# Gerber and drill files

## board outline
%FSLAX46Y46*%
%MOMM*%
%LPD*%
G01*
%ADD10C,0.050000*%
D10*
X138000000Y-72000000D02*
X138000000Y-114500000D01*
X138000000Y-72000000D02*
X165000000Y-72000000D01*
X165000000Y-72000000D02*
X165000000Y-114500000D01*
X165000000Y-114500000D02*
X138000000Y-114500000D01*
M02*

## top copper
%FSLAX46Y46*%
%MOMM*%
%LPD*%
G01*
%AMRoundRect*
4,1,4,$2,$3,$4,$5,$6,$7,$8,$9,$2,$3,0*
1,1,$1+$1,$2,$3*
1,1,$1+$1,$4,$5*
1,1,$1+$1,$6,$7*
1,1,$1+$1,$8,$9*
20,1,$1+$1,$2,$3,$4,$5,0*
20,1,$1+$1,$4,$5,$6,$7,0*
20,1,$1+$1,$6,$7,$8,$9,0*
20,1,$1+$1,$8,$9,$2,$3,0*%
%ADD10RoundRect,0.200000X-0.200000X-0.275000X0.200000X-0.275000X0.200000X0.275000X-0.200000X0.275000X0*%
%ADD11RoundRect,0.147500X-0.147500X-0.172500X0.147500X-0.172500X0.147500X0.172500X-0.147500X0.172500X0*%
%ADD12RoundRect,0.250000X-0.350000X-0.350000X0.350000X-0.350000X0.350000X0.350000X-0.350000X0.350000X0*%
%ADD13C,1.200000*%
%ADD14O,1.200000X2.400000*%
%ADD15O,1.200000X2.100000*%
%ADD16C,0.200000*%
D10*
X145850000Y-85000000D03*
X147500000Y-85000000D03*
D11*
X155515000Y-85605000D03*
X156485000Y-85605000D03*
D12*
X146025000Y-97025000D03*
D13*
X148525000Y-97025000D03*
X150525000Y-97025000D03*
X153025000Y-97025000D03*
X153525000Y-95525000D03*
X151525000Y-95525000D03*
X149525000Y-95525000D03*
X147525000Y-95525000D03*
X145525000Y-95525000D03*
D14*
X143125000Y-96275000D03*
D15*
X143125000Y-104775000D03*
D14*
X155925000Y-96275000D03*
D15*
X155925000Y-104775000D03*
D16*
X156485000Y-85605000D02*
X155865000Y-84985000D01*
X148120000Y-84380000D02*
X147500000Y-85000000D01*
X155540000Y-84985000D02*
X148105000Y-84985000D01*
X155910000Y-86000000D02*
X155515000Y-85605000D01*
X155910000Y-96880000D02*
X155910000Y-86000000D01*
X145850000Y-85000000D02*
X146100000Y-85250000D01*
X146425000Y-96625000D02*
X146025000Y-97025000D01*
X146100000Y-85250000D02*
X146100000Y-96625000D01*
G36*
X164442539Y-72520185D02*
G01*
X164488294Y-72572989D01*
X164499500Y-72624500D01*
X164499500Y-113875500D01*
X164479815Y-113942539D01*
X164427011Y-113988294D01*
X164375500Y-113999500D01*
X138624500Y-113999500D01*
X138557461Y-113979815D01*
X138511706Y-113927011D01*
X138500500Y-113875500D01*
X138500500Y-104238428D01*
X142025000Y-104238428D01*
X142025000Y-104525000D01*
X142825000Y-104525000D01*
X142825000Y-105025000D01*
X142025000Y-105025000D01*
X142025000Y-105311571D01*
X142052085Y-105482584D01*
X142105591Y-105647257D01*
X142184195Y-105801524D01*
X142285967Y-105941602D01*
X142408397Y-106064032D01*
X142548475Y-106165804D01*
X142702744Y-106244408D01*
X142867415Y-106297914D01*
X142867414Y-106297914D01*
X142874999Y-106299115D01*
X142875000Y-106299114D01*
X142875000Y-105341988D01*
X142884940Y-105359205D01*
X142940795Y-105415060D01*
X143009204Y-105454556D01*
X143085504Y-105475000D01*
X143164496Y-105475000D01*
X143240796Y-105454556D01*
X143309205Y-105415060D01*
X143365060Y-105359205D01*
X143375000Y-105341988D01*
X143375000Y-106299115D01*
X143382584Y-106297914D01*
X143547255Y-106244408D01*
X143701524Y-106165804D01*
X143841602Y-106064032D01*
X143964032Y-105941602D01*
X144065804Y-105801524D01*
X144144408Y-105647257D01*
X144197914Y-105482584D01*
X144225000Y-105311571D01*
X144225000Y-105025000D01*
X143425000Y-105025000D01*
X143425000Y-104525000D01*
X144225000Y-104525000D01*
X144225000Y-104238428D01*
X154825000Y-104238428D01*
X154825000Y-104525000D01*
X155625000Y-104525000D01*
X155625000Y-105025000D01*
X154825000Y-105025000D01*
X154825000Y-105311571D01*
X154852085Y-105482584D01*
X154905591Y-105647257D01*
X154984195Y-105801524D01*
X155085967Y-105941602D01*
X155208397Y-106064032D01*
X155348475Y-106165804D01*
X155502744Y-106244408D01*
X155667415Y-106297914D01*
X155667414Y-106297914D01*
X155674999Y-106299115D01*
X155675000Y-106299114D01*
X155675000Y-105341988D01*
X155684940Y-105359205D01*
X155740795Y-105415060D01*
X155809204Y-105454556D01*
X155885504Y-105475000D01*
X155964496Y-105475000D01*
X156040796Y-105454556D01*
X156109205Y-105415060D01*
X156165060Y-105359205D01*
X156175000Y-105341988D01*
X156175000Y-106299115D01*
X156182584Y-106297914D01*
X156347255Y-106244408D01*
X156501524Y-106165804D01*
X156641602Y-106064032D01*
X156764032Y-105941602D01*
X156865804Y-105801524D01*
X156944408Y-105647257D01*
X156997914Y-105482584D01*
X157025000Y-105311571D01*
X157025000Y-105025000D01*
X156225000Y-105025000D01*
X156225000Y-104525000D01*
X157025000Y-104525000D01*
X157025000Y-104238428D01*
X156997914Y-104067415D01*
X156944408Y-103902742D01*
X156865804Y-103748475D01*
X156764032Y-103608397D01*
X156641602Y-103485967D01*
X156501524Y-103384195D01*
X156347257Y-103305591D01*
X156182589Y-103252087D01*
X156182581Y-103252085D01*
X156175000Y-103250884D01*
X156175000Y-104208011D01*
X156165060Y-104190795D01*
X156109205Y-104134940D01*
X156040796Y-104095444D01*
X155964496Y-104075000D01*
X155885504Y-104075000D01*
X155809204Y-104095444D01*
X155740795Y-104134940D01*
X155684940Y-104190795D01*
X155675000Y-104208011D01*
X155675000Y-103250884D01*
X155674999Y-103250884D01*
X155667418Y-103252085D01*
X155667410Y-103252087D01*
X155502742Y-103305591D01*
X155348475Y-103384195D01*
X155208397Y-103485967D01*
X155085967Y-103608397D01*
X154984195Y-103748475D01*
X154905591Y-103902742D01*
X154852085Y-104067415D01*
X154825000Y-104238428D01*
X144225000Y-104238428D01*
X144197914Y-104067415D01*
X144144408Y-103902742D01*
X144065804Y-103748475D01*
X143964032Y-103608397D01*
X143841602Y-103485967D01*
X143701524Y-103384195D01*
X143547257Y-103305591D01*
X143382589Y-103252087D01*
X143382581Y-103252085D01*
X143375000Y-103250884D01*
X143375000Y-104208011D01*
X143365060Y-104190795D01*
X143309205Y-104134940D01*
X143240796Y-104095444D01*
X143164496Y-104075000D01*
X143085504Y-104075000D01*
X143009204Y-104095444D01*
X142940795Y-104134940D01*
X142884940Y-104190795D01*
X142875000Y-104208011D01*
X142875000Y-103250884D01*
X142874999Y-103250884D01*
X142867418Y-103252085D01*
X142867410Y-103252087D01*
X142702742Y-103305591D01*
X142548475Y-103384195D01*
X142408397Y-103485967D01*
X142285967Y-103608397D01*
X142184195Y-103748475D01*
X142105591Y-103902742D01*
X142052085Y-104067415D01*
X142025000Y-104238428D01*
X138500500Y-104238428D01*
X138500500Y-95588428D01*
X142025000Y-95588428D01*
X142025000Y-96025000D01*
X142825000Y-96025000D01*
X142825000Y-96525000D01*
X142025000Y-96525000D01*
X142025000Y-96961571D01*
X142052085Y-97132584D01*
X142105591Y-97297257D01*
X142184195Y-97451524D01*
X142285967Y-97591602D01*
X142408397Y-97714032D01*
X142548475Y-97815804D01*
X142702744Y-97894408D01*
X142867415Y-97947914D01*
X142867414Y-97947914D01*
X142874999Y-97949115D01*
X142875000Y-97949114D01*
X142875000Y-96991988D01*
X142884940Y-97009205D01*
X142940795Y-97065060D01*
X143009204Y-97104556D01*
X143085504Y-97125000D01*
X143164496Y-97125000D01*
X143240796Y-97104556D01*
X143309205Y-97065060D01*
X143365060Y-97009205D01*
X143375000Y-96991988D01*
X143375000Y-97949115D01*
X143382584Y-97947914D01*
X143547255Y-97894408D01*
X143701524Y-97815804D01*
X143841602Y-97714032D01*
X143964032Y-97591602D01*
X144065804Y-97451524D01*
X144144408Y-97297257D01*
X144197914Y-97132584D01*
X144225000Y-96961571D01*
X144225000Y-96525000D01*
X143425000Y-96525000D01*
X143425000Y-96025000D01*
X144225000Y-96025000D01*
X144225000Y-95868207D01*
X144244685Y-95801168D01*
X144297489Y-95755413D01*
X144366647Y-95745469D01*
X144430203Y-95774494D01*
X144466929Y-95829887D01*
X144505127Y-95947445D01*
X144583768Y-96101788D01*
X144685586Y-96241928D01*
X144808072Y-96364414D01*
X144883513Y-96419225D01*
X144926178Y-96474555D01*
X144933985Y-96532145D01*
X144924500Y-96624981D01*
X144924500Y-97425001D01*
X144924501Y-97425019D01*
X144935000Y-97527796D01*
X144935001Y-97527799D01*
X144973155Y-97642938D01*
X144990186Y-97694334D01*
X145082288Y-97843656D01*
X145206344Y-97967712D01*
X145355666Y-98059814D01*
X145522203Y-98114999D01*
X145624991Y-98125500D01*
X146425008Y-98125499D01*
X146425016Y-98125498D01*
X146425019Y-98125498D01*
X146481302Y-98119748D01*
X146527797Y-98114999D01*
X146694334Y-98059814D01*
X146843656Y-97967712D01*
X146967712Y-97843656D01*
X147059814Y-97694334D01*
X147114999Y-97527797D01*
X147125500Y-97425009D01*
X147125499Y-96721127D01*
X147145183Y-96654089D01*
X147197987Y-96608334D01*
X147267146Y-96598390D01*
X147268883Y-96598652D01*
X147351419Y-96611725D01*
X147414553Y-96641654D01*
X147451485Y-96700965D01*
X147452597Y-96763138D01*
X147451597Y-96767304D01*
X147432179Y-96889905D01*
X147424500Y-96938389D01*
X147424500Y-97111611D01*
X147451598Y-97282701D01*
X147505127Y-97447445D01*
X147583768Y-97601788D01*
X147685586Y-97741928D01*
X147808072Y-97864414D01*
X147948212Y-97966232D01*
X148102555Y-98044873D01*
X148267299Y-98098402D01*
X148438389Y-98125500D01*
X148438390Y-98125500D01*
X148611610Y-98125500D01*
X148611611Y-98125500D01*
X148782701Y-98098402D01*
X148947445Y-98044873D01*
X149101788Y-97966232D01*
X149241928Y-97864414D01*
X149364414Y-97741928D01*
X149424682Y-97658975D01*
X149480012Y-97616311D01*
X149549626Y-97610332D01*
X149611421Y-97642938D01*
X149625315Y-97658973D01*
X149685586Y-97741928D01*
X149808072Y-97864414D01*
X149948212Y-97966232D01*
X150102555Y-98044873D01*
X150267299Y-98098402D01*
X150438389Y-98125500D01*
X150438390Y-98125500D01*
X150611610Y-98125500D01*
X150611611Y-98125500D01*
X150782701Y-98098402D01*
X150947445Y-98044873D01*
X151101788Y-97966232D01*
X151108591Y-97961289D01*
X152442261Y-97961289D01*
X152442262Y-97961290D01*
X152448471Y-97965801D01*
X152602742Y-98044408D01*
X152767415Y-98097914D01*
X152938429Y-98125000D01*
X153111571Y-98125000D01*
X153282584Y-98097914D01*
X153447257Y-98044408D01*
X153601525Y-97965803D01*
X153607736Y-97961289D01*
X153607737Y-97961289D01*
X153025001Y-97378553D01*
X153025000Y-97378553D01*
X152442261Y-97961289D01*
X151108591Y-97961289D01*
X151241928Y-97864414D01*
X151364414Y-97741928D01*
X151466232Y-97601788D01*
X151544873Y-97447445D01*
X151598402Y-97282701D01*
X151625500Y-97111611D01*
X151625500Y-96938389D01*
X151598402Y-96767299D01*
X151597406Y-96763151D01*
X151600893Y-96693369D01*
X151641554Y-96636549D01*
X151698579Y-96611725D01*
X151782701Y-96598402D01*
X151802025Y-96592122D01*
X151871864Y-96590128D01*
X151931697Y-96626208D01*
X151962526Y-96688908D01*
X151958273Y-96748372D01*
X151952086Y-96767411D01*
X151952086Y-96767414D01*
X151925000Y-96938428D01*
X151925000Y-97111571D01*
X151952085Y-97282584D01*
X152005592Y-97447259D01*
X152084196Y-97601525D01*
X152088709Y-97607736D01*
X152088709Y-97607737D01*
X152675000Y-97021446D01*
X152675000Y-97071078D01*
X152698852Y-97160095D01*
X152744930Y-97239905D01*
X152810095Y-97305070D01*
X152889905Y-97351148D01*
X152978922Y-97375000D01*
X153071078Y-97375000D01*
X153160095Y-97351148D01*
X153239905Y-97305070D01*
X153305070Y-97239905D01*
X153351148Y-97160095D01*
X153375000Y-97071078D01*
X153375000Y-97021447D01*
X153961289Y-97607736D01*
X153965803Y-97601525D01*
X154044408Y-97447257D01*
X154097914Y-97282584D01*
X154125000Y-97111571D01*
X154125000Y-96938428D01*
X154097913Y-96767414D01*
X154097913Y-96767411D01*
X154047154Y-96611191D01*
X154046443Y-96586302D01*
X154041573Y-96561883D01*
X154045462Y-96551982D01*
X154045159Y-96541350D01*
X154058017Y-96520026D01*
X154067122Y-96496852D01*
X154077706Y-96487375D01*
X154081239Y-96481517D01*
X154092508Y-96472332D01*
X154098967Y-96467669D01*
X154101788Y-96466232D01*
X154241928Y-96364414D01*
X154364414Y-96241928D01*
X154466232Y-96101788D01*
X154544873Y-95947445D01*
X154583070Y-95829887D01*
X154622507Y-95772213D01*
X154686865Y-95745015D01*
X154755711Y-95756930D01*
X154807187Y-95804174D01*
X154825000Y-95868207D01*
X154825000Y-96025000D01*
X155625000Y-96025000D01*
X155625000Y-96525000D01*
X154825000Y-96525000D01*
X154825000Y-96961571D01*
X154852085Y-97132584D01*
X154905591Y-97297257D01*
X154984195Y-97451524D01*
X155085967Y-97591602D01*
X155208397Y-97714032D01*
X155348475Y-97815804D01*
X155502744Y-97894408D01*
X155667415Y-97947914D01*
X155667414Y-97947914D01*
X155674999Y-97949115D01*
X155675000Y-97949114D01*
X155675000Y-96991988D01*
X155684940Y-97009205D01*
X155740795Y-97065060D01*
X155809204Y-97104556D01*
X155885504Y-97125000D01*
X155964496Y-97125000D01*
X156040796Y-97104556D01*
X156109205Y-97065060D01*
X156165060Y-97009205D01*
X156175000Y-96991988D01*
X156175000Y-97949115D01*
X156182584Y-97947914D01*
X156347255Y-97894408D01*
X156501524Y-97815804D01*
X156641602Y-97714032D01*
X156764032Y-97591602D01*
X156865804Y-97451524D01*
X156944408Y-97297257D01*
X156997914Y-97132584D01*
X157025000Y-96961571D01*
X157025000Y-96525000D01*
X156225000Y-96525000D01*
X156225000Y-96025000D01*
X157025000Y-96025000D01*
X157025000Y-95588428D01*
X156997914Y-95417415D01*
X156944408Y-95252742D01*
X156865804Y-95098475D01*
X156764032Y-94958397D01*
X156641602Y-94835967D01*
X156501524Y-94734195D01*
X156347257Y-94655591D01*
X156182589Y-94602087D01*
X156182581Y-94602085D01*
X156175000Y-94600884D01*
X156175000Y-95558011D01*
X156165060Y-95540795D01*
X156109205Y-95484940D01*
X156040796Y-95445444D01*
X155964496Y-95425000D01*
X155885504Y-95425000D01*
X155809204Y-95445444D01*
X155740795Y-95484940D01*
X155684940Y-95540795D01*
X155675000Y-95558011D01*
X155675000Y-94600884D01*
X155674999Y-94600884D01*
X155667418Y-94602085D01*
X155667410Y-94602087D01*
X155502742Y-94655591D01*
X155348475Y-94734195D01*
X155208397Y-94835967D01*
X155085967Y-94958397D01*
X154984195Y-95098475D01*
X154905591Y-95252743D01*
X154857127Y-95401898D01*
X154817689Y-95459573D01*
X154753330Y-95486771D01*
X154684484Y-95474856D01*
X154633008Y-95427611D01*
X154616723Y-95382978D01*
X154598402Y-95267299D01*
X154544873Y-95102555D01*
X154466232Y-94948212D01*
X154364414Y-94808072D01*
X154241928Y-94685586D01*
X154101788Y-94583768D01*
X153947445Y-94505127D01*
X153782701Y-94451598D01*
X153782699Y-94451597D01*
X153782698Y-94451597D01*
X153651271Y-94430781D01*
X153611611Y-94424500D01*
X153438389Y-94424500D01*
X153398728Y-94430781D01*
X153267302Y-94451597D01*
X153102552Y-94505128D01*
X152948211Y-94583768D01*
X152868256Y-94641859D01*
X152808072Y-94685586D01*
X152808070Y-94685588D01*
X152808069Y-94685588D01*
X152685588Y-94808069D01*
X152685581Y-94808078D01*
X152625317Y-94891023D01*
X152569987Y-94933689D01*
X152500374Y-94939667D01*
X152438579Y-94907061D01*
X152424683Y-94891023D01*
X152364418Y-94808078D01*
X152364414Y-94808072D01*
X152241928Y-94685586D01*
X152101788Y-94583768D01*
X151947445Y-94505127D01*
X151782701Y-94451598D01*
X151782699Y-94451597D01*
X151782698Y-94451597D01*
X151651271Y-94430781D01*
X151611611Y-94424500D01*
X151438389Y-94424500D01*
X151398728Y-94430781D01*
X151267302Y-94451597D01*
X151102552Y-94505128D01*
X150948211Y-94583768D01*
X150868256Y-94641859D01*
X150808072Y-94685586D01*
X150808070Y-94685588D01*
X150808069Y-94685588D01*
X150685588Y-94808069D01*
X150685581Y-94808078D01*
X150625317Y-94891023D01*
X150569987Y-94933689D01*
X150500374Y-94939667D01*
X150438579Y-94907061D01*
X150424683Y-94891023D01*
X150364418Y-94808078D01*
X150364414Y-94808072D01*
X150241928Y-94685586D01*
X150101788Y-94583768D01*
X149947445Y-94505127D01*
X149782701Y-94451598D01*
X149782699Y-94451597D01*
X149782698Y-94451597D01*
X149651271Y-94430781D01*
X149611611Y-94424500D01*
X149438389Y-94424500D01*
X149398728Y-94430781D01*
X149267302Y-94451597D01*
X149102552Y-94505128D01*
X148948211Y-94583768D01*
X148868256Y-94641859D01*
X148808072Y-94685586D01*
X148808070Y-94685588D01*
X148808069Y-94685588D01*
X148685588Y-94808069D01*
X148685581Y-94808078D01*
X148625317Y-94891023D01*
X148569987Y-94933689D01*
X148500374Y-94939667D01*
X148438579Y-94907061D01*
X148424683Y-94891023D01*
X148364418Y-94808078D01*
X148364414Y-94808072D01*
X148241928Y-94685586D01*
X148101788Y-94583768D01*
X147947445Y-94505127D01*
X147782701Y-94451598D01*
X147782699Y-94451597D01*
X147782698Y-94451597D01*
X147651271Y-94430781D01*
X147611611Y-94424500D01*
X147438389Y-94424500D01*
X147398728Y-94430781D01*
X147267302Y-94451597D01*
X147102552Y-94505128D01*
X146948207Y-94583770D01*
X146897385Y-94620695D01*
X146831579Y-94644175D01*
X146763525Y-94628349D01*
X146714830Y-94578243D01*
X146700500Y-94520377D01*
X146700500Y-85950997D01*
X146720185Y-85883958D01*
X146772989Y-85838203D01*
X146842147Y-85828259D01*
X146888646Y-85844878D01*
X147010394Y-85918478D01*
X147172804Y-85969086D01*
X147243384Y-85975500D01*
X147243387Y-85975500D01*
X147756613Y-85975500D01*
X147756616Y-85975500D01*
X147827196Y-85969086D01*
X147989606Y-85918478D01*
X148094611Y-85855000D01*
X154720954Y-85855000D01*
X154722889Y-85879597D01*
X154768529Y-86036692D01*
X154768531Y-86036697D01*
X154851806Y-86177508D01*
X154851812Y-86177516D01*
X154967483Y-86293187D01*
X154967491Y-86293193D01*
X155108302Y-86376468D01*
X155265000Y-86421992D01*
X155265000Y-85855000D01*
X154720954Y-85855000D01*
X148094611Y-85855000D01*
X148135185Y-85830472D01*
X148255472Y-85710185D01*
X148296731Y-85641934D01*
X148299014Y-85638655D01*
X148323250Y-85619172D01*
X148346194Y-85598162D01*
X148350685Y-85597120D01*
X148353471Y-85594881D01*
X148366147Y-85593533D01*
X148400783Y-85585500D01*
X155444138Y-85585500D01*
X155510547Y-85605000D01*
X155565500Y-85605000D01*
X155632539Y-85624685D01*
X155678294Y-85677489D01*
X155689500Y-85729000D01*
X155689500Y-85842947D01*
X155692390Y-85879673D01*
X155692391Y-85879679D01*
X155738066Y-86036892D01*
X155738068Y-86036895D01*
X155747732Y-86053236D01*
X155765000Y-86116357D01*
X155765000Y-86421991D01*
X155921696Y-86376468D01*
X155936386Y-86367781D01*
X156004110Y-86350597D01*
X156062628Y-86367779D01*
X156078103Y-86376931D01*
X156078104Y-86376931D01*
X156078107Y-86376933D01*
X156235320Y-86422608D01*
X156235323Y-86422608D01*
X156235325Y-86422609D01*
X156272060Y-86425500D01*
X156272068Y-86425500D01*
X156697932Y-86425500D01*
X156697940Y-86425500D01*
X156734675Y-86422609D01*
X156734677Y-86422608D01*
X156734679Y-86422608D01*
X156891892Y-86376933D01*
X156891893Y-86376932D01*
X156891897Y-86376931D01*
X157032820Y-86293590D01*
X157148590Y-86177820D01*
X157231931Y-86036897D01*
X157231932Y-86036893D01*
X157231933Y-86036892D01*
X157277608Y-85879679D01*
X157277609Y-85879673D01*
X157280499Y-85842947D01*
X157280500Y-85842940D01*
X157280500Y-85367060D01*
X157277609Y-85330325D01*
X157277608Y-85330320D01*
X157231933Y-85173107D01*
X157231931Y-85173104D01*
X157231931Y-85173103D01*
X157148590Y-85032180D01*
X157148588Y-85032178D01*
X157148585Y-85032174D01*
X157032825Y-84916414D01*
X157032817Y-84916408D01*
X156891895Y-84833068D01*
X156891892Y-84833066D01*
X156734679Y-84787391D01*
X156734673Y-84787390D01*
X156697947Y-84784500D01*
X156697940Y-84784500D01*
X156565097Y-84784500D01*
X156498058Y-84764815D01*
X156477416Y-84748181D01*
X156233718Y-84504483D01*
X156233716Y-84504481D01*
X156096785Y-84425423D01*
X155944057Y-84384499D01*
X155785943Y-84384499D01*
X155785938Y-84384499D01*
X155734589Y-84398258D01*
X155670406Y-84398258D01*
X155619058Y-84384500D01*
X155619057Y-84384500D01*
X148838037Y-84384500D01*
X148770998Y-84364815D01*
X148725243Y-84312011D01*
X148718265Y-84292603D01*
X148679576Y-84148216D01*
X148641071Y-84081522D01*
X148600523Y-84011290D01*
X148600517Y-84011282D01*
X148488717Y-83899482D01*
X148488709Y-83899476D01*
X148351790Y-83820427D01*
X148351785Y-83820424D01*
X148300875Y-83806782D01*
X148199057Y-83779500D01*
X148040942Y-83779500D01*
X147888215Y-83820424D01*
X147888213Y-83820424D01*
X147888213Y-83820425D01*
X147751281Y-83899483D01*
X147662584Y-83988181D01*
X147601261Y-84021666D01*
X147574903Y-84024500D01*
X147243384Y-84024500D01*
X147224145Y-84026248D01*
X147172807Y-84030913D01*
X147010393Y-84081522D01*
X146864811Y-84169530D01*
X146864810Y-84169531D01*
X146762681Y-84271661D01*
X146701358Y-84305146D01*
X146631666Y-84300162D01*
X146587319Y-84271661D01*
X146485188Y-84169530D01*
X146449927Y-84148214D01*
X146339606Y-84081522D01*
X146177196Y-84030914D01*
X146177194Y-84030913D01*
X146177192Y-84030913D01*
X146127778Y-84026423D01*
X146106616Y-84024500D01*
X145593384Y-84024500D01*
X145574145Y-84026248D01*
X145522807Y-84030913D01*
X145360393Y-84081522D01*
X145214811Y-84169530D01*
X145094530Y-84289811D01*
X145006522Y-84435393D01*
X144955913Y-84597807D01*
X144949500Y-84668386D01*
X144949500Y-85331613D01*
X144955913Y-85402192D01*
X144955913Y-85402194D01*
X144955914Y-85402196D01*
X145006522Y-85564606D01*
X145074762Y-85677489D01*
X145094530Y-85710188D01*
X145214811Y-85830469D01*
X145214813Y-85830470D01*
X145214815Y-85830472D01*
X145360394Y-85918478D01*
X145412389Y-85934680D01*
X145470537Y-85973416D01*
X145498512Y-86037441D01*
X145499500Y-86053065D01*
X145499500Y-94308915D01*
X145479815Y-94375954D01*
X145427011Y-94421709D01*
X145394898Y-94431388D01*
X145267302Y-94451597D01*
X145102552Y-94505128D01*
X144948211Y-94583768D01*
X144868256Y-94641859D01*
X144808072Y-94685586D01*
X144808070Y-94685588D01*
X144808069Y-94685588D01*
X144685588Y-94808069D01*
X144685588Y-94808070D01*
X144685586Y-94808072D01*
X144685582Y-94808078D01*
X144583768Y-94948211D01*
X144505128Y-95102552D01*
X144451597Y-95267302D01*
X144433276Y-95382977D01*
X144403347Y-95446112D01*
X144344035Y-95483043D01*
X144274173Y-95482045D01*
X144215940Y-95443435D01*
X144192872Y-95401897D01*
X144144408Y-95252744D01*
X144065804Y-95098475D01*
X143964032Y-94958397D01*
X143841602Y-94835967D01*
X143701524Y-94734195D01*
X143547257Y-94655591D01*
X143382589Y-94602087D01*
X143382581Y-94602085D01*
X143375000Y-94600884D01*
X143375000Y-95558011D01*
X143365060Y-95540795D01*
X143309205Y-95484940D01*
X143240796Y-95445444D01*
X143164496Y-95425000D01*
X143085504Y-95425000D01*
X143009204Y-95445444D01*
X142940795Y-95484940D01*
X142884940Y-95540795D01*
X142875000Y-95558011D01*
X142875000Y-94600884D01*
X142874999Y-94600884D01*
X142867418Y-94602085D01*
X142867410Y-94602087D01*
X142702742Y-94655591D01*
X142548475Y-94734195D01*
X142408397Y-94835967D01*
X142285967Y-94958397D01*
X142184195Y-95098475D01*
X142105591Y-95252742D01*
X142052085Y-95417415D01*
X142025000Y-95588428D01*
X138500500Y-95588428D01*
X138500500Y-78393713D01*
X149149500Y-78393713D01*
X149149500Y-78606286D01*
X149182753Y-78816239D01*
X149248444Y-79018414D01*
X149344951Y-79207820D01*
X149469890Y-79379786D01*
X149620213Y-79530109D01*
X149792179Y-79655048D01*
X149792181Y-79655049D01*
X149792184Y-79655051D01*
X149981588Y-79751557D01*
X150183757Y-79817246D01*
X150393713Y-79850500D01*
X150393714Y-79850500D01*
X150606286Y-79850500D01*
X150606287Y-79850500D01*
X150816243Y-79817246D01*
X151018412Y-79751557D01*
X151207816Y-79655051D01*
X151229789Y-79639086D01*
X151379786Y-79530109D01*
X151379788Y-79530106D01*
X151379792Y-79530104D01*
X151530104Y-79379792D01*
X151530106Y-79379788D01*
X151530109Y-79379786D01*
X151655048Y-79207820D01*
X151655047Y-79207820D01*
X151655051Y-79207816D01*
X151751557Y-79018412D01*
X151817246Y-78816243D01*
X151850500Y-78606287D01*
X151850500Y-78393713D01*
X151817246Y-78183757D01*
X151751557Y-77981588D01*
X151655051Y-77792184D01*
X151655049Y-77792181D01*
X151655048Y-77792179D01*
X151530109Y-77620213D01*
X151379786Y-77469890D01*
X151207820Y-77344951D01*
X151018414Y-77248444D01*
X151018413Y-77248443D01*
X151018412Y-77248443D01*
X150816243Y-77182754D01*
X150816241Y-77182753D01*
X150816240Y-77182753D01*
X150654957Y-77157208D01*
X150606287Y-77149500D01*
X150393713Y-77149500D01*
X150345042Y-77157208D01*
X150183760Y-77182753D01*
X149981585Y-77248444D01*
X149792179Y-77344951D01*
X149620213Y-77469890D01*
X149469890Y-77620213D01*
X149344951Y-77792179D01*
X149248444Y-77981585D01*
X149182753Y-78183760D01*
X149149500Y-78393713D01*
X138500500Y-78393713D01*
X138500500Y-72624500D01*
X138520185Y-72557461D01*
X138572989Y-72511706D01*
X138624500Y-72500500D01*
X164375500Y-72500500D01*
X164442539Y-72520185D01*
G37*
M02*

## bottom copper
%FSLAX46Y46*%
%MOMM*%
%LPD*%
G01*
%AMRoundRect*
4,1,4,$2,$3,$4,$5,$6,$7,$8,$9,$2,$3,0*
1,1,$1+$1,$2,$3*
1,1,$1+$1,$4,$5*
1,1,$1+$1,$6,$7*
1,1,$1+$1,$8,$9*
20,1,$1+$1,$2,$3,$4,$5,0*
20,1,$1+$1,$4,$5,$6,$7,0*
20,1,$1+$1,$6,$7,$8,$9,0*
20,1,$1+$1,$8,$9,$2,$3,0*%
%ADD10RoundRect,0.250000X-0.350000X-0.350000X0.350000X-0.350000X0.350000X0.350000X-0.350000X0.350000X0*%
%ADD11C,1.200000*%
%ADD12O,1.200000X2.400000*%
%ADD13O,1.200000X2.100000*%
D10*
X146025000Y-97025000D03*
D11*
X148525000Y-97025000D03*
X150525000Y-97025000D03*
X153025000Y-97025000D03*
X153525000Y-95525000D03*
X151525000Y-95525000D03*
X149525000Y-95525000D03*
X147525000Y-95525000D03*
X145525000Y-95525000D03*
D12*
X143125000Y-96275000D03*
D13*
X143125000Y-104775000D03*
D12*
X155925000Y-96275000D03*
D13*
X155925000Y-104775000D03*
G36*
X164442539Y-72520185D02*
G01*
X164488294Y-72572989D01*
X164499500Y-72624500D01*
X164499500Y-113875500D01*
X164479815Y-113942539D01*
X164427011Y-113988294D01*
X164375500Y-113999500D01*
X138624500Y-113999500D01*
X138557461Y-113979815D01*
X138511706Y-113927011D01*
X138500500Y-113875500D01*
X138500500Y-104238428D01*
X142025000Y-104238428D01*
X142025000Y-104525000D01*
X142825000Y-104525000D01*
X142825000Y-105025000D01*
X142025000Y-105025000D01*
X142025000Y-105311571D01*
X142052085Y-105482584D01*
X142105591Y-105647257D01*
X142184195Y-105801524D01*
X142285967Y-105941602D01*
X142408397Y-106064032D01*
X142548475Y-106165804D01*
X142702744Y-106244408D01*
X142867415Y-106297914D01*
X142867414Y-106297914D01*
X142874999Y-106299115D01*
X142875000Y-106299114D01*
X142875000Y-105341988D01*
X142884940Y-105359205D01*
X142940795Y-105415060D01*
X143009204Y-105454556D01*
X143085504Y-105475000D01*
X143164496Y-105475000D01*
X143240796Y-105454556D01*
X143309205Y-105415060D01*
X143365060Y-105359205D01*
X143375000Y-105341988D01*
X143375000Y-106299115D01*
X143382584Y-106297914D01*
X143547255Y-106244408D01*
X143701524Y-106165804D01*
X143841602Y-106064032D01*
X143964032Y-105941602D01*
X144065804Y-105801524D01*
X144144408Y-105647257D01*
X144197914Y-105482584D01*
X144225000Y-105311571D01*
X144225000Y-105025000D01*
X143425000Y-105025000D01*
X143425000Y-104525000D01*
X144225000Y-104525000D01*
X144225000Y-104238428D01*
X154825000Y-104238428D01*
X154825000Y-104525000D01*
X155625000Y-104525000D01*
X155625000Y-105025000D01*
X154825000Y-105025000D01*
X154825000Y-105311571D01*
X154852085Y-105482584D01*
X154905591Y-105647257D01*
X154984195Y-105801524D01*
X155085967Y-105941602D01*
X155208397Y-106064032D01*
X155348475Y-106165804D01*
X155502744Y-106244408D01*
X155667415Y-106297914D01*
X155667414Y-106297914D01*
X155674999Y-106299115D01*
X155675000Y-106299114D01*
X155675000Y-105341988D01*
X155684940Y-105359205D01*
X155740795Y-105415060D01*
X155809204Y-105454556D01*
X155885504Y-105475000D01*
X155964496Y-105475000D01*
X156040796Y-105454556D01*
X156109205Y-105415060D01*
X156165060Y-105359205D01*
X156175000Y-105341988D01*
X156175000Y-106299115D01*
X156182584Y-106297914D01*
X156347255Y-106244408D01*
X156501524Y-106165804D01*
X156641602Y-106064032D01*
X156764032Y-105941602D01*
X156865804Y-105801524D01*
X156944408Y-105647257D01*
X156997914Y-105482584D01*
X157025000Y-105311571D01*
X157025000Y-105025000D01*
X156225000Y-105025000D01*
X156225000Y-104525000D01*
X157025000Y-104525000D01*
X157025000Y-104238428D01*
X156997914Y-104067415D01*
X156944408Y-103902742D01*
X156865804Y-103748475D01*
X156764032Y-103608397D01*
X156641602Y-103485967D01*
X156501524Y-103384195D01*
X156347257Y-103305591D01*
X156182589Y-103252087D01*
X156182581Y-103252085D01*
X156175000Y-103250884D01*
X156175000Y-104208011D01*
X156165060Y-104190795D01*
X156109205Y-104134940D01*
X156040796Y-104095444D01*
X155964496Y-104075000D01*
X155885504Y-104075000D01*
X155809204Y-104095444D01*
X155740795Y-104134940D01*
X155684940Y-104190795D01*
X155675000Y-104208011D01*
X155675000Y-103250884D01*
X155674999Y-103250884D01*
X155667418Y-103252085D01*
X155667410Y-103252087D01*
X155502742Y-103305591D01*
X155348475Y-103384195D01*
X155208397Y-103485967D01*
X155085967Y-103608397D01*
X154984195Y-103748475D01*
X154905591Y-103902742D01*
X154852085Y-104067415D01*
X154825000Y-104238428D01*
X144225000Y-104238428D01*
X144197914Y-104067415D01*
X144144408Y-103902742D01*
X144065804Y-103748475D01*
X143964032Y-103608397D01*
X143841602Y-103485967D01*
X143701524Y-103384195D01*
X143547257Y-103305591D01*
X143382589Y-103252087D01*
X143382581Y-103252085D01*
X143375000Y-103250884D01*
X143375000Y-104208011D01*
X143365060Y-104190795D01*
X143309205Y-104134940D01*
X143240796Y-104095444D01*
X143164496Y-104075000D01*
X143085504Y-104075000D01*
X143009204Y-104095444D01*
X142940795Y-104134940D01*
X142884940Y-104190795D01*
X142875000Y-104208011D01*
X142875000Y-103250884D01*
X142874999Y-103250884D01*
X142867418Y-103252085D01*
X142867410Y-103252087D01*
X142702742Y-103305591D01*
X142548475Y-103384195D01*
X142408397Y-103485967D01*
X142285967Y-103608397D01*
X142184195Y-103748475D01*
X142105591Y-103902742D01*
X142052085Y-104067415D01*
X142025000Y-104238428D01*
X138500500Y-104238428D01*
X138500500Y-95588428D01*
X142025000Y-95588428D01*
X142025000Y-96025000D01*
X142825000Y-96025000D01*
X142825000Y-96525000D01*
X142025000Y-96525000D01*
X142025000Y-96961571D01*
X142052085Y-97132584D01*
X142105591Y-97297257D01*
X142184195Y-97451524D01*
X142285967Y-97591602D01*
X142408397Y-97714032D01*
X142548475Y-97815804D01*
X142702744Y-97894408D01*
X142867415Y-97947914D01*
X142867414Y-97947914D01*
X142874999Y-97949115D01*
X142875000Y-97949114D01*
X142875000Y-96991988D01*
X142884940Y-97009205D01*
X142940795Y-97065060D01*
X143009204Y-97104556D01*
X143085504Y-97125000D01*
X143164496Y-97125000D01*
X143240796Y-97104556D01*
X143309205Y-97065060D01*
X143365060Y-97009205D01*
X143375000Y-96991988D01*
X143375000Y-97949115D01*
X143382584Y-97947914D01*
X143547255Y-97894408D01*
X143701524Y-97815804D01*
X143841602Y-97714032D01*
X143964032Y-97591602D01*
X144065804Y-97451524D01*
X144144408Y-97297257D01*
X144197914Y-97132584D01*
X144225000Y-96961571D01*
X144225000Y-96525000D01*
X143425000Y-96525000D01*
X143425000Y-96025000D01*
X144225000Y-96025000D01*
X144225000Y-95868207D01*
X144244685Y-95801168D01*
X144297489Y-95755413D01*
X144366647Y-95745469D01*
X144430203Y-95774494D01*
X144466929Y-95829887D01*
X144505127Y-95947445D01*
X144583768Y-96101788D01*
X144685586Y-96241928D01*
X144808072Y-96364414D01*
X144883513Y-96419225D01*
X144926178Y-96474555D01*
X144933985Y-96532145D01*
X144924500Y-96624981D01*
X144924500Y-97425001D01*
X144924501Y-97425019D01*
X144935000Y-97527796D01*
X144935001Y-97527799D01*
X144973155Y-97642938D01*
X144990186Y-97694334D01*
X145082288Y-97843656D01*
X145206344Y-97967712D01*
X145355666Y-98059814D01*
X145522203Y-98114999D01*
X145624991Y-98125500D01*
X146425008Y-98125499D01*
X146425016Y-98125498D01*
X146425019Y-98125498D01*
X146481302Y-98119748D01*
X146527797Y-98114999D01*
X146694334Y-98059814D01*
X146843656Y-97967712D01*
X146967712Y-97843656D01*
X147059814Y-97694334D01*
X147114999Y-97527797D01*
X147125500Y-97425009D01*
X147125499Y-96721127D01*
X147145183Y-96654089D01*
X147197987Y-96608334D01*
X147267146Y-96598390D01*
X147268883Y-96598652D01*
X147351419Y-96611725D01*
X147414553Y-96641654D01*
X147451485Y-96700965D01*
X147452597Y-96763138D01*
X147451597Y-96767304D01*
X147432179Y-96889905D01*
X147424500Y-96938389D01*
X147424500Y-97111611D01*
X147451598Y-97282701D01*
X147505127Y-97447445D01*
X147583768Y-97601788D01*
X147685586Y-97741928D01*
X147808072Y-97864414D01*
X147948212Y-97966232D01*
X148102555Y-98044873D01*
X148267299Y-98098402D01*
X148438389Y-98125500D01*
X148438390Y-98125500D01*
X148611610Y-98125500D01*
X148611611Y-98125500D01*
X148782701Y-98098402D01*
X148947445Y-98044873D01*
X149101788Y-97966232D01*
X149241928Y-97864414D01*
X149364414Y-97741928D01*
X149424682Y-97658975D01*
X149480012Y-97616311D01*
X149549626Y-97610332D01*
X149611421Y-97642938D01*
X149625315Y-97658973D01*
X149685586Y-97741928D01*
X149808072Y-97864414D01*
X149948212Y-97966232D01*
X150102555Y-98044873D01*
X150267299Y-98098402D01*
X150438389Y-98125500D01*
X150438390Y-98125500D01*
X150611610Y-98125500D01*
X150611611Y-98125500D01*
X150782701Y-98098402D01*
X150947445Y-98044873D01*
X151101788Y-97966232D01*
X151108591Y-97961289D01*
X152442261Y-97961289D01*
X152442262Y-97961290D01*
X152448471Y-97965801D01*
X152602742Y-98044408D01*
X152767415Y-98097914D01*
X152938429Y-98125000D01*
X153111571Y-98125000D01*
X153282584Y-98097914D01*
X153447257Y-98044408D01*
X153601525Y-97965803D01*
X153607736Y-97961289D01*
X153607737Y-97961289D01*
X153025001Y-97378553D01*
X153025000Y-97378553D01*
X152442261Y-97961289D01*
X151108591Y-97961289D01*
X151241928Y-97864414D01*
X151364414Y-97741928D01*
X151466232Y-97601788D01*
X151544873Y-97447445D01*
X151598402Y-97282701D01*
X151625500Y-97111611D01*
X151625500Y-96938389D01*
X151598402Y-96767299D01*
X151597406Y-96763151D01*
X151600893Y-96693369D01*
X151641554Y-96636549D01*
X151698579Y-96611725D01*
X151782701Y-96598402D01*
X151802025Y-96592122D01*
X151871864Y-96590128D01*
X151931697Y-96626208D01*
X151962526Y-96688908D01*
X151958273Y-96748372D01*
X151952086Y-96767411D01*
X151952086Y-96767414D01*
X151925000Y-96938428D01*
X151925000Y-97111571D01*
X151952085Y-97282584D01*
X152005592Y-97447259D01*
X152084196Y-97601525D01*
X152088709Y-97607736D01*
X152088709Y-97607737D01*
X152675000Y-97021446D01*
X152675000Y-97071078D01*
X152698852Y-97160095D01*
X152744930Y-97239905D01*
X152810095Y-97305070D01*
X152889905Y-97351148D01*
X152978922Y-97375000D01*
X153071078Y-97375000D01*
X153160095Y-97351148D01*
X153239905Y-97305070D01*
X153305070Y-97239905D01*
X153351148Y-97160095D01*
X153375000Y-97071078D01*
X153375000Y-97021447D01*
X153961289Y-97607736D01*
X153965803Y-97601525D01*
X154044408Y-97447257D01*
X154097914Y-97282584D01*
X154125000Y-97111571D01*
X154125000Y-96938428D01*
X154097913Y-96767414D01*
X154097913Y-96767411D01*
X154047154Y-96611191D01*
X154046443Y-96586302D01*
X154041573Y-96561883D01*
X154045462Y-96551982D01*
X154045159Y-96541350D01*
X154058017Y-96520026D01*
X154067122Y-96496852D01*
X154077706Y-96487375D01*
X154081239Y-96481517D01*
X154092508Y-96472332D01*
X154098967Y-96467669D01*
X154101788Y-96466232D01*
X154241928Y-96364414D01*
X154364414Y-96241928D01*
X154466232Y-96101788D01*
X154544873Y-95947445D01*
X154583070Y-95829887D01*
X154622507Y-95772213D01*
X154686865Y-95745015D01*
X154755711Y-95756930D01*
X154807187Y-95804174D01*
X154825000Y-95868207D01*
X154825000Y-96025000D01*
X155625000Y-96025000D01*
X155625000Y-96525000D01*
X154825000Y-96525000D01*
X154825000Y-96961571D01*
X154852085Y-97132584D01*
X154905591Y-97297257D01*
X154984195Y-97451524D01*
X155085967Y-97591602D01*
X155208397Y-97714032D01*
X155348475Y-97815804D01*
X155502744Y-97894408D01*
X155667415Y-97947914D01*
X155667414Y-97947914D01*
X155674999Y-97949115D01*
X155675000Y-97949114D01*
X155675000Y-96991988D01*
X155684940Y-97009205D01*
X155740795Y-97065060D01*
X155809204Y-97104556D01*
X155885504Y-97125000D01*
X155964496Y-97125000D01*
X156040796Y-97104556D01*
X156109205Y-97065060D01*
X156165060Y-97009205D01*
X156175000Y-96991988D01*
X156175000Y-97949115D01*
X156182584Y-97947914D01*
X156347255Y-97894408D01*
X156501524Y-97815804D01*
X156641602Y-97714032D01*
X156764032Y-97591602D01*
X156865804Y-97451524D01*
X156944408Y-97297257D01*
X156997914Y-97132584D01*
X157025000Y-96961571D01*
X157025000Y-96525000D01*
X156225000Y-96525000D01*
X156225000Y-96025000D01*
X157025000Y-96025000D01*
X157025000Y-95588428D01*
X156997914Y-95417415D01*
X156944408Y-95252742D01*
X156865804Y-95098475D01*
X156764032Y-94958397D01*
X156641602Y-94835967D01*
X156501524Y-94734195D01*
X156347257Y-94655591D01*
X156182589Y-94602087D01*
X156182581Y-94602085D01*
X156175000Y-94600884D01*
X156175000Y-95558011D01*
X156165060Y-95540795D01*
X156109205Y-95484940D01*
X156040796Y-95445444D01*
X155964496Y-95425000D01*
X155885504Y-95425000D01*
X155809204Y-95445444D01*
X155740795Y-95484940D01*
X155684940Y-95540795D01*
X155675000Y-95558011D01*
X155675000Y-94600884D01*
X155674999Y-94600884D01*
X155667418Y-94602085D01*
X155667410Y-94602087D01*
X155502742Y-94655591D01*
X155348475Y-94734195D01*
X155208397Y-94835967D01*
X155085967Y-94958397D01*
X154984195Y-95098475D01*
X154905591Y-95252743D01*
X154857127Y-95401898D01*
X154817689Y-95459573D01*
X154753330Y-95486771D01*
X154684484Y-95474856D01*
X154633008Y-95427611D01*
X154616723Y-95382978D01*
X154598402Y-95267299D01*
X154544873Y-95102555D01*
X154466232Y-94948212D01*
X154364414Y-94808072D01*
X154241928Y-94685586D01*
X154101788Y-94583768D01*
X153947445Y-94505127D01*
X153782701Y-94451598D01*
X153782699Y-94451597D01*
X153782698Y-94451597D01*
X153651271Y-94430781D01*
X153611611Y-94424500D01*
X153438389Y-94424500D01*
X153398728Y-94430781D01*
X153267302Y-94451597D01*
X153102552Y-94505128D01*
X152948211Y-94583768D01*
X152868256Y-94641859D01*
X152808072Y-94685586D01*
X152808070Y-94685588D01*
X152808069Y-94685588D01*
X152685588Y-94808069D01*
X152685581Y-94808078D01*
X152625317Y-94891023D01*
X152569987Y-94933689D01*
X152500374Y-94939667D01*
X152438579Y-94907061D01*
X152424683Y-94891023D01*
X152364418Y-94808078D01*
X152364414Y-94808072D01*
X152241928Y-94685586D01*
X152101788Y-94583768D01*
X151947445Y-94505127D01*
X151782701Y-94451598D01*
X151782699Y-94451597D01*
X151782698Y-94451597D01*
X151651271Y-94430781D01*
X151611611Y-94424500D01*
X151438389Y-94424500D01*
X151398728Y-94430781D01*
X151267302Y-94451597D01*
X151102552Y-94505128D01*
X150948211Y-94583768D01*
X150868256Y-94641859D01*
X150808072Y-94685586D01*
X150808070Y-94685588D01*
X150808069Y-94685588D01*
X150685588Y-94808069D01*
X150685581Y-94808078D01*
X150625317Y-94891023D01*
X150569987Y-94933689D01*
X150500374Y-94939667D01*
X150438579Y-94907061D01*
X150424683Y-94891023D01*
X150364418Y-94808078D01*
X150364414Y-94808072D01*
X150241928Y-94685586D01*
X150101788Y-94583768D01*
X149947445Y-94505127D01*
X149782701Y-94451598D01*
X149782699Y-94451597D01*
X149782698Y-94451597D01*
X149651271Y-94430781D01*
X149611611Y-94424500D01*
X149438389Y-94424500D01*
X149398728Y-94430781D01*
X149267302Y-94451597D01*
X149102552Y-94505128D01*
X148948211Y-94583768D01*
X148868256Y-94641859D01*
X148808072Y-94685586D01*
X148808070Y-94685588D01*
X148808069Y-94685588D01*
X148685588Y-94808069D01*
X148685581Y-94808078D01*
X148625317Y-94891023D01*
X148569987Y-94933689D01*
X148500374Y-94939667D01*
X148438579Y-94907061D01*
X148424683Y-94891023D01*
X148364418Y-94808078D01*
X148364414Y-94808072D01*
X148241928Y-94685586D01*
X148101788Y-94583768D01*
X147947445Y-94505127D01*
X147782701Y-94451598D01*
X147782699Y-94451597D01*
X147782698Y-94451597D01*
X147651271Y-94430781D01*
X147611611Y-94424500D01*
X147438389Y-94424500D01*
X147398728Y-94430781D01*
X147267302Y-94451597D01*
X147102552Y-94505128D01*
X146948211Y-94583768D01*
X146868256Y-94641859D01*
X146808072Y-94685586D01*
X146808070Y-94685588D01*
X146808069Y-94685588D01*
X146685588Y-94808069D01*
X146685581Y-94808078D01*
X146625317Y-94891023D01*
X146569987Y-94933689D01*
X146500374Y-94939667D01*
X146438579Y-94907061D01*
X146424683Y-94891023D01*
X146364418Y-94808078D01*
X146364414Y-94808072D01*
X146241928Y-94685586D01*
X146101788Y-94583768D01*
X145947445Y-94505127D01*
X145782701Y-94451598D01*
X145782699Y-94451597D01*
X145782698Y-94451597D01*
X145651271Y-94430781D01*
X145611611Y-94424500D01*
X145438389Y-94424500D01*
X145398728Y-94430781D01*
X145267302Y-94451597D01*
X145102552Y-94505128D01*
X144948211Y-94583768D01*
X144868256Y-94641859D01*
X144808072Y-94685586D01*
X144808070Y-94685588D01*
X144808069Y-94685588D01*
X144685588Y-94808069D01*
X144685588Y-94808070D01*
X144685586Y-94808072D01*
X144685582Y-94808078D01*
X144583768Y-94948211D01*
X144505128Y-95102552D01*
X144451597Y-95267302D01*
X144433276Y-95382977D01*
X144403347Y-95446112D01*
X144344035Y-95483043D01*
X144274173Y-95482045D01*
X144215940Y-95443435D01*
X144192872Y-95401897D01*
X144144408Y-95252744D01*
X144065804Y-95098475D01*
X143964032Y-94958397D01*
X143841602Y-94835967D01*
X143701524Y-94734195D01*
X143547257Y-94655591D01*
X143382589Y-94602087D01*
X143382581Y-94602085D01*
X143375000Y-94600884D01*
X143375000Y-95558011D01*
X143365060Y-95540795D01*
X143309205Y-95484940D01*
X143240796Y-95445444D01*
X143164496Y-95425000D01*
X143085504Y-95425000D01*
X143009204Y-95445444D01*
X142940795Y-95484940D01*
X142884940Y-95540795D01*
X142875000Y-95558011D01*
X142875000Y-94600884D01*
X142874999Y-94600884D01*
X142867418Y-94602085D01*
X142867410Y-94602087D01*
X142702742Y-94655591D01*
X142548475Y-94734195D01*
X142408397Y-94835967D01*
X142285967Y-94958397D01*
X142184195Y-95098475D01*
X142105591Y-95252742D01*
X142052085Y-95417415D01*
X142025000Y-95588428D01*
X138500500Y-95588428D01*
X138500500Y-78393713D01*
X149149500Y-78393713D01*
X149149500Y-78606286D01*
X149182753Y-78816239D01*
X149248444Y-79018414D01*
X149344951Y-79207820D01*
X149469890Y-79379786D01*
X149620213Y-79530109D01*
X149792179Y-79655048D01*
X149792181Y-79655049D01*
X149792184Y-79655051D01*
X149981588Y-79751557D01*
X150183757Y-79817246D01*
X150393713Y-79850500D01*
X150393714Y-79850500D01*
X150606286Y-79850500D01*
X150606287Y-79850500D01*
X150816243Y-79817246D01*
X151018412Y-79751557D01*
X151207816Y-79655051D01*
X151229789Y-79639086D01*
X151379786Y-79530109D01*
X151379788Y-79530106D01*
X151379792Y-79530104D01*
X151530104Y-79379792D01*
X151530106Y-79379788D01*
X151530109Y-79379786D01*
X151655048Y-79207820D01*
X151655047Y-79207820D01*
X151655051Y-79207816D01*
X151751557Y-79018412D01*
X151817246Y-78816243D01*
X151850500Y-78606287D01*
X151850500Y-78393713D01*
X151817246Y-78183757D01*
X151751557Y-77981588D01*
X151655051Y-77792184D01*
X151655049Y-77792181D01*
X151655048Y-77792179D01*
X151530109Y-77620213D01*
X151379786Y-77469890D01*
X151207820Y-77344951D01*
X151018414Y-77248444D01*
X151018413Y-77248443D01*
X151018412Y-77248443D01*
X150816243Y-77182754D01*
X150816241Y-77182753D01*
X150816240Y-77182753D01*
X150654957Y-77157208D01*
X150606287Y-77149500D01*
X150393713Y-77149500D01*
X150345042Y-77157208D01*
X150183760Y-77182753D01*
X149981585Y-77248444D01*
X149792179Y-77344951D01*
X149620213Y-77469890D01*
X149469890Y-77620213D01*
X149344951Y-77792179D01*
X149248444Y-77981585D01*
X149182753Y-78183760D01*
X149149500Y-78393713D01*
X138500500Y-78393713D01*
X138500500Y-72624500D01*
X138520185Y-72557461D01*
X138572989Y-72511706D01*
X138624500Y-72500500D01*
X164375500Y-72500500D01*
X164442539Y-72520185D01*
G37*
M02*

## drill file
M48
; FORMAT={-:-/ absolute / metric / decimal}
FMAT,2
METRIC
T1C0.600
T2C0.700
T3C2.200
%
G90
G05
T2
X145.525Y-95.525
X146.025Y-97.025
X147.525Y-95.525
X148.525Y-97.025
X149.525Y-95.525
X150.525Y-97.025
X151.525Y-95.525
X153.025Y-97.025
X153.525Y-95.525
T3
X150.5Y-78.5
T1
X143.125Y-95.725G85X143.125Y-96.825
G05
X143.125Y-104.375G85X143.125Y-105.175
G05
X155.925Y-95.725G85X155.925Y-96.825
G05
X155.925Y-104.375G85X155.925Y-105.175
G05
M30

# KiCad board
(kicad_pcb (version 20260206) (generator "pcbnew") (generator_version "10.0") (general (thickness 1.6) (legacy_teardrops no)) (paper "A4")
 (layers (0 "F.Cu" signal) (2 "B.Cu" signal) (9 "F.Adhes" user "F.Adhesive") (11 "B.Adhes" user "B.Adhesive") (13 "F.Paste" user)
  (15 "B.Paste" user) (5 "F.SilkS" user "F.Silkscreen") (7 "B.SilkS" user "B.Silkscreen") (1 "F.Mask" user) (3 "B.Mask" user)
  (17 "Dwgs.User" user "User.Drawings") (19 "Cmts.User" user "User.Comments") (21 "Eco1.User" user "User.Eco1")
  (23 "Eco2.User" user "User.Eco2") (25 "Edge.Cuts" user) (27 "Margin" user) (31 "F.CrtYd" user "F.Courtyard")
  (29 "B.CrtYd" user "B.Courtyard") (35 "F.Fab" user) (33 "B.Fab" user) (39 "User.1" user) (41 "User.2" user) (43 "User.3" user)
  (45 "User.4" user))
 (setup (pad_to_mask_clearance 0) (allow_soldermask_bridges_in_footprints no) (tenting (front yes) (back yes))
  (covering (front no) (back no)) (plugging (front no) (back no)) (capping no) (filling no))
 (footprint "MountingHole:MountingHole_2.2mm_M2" (layer "F.Cu") (at 150.5 78.5)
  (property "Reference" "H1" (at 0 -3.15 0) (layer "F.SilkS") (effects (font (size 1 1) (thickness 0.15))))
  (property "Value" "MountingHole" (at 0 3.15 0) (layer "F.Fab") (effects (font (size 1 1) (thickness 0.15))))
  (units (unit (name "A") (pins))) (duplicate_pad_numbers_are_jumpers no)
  (pad "" np_thru_hole circle (at 0 0) (size 2.2 2.2) (drill 2.2) (layers "*.Cu" "*.Mask")))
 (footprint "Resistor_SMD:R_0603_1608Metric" (layer "F.Cu") (at 146.675 85)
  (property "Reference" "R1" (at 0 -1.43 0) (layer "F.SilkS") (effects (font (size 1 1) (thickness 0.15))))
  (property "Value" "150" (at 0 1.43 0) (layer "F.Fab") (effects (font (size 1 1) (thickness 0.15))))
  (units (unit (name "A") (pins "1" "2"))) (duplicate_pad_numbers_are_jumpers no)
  (pad "1" smd roundrect (at -0.825 0) (size 0.8 0.95) (layers "F.Cu" "F.Mask" "F.Paste") (roundrect_rratio 0.25)
   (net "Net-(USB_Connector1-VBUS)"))
  (pad "2" smd roundrect (at 0.825 0) (size 0.8 0.95) (layers "F.Cu" "F.Mask" "F.Paste") (roundrect_rratio 0.25) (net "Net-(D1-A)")))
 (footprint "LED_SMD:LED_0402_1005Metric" (layer "F.Cu") (at 156 85.605)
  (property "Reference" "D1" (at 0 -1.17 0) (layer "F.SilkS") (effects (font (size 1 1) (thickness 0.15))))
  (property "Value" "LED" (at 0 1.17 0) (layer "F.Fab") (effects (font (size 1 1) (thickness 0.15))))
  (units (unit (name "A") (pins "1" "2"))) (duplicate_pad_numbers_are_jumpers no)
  (pad "1" smd roundrect (at -0.485 0) (size 0.59 0.64) (layers "F.Cu" "F.Mask" "F.Paste") (roundrect_rratio 0.25) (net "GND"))
  (pad "2" smd roundrect (at 0.485 0) (size 0.59 0.64) (layers "F.Cu" "F.Mask" "F.Paste") (roundrect_rratio 0.25) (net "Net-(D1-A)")))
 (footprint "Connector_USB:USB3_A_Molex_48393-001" (layer "F.Cu") (at 146.025 97.025)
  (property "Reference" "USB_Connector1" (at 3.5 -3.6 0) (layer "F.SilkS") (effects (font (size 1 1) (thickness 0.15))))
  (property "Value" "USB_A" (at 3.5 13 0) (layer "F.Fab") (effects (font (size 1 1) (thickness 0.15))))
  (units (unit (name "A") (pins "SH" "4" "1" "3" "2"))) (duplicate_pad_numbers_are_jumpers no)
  (pad "1" thru_hole roundrect (at 0 0) (size 1.2 1.2) (drill 0.7) (layers "*.Cu" "*.Mask") (remove_unused_layers no)
   (roundrect_rratio 0.2083333333) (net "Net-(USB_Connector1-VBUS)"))
  (pad "2" thru_hole circle (at 2.5 0) (size 1.2 1.2) (drill 0.7) (layers "*.Cu" "*.Mask") (remove_unused_layers no)
   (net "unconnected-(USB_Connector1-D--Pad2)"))
  (pad "3" thru_hole circle (at 4.5 0) (size 1.2 1.2) (drill 0.7) (layers "*.Cu" "*.Mask") (remove_unused_layers no)
   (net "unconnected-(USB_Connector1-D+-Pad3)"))
  (pad "4" thru_hole circle (at 7 0) (size 1.2 1.2) (drill 0.7) (layers "*.Cu" "*.Mask") (remove_unused_layers no) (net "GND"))
  (pad "5" thru_hole circle (at 7.5 -1.5) (size 1.2 1.2) (drill 0.7) (layers "*.Cu" "*.Mask") (remove_unused_layers no))
  (pad "6" thru_hole circle (at 5.5 -1.5) (size 1.2 1.2) (drill 0.7) (layers "*.Cu" "*.Mask") (remove_unused_layers no))
  (pad "7" thru_hole circle (at 3.5 -1.5) (size 1.2 1.2) (drill 0.7) (layers "*.Cu" "*.Mask") (remove_unused_layers no))
  (pad "8" thru_hole circle (at 1.5 -1.5) (size 1.2 1.2) (drill 0.7) (layers "*.Cu" "*.Mask") (remove_unused_layers no))
  (pad "9" thru_hole circle (at -0.5 -1.5) (size 1.2 1.2) (drill 0.7) (layers "*.Cu" "*.Mask") (remove_unused_layers no))
  (pad "SH" thru_hole oval (at -2.9 -0.75) (size 1.2 2.4) (drill oval 0.6 1.7) (layers "*.Cu" "*.Mask") (remove_unused_layers no)
   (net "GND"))
  (pad "SH" thru_hole oval (at -2.9 7.75) (size 1.2 2.1) (drill oval 0.6 1.4) (layers "*.Cu" "*.Mask") (remove_unused_layers no) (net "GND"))
  (pad "SH" thru_hole oval (at 9.9 -0.75) (size 1.2 2.4) (drill oval 0.6 1.7) (layers "*.Cu" "*.Mask") (remove_unused_layers no) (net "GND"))
  (pad "SH" thru_hole oval (at 9.9 7.75) (size 1.2 2.1) (drill oval 0.6 1.4) (layers "*.Cu" "*.Mask") (remove_unused_layers no) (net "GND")))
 (gr_line (start 138 72) (end 138 114.5) (stroke (width 0.05) (type default)) (layer "Edge.Cuts"))
 (gr_line (start 138 72) (end 165 72) (stroke (width 0.05) (type default)) (layer "Edge.Cuts"))
 (gr_line (start 165 72) (end 165 114.5) (stroke (width 0.05) (type default)) (layer "Edge.Cuts"))
 (gr_line (start 165 114.5) (end 138 114.5) (stroke (width 0.05) (type default)) (layer "Edge.Cuts"))
 (segment (start 156.485 85.605) (end 155.865 84.985) (width 0.2) (layer "F.Cu") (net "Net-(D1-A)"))
 (segment (start 148.12 84.38) (end 147.5 85) (width 0.2) (layer "F.Cu") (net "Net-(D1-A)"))
 (segment (start 155.54 84.985) (end 148.105 84.985) (width 0.2) (layer "F.Cu") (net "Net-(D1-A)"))
 (segment (start 155.91 86) (end 155.515 85.605) (width 0.2) (layer "F.Cu") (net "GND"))
 (segment (start 155.91 96.88) (end 155.91 86) (width 0.2) (layer "F.Cu") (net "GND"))
 (segment (start 145.85 85) (end 146.1 85.25) (width 0.2) (layer "F.Cu") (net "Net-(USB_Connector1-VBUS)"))
 (segment (start 146.425 96.625) (end 146.025 97.025) (width 0.2) (layer "F.Cu") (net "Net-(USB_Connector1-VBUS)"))
 (segment (start 146.1 85.25) (end 146.1 96.625) (width 0.2) (layer "F.Cu") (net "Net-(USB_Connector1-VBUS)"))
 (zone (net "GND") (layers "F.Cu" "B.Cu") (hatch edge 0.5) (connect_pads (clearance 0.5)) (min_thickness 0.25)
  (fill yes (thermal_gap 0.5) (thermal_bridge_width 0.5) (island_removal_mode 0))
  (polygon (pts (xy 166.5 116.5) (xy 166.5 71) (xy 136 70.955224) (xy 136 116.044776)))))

